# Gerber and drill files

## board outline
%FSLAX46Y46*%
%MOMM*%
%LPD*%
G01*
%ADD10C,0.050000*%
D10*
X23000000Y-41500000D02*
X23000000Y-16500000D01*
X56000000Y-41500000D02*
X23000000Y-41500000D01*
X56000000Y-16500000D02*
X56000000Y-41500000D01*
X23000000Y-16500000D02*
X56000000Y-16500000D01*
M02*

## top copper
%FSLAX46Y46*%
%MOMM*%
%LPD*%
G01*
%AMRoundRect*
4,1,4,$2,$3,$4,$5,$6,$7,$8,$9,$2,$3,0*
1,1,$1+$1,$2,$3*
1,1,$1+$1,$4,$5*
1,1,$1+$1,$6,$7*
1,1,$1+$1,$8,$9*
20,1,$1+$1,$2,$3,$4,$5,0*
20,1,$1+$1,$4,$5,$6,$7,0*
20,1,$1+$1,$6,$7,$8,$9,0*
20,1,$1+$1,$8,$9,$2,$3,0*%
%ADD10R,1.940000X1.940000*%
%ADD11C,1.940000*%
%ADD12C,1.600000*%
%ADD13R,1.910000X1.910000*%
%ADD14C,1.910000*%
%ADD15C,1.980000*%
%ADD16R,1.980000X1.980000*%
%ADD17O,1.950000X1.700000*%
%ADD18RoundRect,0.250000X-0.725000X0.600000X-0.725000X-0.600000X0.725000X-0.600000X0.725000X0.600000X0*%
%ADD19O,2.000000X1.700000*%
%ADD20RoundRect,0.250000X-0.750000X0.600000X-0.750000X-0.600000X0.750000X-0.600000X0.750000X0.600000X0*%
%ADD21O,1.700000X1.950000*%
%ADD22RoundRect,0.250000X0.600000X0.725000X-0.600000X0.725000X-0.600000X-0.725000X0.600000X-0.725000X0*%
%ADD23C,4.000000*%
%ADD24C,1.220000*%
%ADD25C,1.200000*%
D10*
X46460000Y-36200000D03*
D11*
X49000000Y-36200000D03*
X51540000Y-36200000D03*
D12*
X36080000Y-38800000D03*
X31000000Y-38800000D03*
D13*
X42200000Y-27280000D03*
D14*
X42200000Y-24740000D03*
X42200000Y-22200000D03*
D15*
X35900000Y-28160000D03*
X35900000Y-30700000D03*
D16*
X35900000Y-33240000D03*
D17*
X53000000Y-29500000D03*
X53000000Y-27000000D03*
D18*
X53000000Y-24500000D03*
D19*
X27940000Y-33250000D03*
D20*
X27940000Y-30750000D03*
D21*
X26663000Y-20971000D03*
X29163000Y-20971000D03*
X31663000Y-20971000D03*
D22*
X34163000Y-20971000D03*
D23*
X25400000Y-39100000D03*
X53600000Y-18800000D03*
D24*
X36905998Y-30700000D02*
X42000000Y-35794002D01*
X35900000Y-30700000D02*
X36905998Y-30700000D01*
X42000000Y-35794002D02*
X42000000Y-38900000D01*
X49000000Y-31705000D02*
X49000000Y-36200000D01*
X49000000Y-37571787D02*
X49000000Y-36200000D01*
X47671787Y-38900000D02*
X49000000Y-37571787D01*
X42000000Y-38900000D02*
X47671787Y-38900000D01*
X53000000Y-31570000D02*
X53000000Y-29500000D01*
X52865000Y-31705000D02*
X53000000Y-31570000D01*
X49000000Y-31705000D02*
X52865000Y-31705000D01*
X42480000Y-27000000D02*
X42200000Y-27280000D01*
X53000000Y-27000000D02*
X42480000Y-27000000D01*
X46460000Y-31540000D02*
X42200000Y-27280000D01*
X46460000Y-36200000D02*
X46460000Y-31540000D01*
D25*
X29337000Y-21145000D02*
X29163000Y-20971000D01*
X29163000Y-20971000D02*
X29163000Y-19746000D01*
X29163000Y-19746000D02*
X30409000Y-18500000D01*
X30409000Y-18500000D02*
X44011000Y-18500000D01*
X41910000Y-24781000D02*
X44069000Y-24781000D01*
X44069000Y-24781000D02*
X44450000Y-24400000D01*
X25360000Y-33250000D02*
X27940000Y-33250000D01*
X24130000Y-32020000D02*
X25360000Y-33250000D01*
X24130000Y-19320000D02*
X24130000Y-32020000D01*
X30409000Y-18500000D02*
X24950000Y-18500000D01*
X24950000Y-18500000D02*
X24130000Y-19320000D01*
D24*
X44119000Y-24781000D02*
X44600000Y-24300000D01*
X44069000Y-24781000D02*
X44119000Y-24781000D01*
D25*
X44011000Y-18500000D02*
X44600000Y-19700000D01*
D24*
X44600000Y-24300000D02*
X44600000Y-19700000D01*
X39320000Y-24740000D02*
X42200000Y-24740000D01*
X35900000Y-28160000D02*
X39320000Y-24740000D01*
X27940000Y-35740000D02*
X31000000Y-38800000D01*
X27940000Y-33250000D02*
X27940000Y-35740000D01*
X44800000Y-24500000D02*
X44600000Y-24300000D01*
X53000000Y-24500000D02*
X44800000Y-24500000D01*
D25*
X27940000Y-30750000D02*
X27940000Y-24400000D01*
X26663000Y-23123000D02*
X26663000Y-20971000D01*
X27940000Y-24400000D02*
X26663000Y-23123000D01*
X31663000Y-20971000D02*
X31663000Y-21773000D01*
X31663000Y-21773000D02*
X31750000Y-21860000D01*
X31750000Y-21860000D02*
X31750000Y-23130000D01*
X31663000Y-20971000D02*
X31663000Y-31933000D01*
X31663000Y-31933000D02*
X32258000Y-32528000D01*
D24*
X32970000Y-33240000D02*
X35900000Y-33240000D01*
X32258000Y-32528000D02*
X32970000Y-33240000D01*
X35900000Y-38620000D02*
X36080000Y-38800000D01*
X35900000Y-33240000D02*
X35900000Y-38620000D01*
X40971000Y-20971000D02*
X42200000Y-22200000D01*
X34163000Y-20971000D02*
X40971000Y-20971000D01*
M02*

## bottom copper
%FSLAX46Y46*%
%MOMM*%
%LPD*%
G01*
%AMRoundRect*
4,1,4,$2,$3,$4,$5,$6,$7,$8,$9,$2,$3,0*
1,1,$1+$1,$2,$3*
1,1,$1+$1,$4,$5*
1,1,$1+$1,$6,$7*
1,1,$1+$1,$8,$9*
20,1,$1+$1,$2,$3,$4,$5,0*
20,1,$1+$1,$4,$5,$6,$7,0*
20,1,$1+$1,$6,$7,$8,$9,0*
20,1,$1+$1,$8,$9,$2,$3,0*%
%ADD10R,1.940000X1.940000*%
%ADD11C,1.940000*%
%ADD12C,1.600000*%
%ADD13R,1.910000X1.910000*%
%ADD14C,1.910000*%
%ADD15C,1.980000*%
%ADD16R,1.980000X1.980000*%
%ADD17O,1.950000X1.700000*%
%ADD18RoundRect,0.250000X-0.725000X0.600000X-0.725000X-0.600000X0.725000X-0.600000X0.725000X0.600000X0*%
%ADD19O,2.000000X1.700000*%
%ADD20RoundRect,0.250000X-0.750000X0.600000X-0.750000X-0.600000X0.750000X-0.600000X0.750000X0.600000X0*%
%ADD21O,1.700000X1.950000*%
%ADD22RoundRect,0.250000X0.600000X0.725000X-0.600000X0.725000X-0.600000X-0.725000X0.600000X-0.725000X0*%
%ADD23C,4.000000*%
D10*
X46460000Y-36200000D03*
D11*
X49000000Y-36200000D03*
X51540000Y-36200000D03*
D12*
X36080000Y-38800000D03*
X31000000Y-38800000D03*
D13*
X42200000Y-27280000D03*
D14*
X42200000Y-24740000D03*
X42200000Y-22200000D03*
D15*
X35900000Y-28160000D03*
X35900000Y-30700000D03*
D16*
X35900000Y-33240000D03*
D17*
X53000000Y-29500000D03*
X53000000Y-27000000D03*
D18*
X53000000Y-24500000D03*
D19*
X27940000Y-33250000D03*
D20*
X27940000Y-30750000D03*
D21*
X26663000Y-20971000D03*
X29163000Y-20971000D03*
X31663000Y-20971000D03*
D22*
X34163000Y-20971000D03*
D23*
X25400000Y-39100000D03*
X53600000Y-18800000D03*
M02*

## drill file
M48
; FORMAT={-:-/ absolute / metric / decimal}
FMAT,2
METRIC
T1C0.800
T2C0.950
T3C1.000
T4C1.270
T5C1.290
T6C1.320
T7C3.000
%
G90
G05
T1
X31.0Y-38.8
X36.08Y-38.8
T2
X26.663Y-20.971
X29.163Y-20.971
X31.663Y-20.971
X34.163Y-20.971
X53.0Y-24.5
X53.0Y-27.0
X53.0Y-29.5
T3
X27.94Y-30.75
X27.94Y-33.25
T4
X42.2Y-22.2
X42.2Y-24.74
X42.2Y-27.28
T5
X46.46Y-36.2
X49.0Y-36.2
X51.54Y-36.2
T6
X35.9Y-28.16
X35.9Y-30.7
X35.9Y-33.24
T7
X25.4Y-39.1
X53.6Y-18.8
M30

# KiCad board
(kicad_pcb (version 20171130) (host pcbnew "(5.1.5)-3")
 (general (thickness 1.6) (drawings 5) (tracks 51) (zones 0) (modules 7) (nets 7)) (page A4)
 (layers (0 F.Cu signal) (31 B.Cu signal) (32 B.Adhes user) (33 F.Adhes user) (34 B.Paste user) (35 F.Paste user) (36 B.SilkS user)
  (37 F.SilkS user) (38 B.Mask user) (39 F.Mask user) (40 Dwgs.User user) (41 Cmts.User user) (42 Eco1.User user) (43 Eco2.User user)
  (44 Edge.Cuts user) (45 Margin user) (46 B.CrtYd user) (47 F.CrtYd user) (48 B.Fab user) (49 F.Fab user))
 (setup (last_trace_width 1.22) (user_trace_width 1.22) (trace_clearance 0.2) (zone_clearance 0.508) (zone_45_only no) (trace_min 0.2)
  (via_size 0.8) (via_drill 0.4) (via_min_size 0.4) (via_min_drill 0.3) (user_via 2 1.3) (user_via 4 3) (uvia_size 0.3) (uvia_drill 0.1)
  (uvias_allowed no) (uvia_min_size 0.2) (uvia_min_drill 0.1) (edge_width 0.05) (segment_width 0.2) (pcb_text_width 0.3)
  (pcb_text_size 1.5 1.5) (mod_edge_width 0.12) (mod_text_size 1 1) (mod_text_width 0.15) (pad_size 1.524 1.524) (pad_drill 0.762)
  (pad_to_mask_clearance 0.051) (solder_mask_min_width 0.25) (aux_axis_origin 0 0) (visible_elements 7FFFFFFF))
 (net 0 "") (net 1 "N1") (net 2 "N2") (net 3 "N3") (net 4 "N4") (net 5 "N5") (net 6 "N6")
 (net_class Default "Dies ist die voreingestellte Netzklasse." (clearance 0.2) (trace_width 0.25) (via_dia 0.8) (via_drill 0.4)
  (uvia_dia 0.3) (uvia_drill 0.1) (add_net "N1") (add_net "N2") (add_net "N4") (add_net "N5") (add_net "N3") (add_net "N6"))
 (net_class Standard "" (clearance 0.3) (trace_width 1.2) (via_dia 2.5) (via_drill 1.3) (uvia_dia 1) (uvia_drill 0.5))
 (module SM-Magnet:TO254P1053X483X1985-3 (layer F.Cu) (at 49 36.2)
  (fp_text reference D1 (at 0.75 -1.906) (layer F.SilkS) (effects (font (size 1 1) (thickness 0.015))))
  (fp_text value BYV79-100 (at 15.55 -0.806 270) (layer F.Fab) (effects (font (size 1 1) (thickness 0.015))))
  (pad 1 thru_hole rect (at -2.54 0) (size 1.94 1.94) (drill 1.29) (layers *.Cu *.Mask) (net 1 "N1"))
  (pad 2 thru_hole circle (at 0 0) (size 1.94 1.94) (drill 1.29) (layers *.Cu *.Mask) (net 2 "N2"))
  (pad 3 thru_hole circle (at 2.54 0) (size 1.94 1.94) (drill 1.29) (layers *.Cu *.Mask)))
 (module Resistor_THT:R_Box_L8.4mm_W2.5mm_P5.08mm (layer F.Cu) (at 31 38.8)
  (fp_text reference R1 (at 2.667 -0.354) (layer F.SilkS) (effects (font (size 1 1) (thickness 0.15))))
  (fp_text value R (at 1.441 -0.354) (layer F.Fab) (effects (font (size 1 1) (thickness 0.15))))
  (pad 2 thru_hole circle (at 5.08 0) (size 1.6 1.6) (drill 0.8) (layers *.Cu *.Mask) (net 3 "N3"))
  (pad 1 thru_hole circle (at 0 0) (size 1.6 1.6) (drill 0.8) (layers *.Cu *.Mask) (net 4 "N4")))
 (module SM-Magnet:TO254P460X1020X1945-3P (layer F.Cu) (at 42.2 24.74 180)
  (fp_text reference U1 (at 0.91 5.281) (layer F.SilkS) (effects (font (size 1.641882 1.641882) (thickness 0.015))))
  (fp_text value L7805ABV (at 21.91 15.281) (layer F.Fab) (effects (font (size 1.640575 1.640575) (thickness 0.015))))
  (pad 1 thru_hole rect (at 0 -2.54 180) (size 1.91 1.91) (drill 1.27) (layers *.Cu *.Mask) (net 1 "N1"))
  (pad 2 thru_hole circle (at 0 0 180) (size 1.91 1.91) (drill 1.27) (layers *.Cu *.Mask) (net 4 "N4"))
  (pad 3 thru_hole circle (at 0 2.54 180) (size 1.91 1.91) (drill 1.27) (layers *.Cu *.Mask) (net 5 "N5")))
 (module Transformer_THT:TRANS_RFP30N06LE (layer F.Cu) (at 35.9 30.7 90)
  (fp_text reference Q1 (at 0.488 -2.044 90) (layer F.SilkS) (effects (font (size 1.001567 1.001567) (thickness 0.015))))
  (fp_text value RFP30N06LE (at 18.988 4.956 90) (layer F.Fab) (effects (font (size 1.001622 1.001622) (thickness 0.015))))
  (pad 3 thru_hole circle (at 2.54 0 90) (size 1.98 1.98) (drill 1.32) (layers *.Cu *.Mask) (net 4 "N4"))
  (pad 2 thru_hole circle (at 0 0 90) (size 1.98 1.98) (drill 1.32) (layers *.Cu *.Mask) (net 2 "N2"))
  (pad 1 thru_hole rect (at -2.54 0 90) (size 1.98 1.98) (drill 1.32) (layers *.Cu *.Mask) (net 3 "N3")))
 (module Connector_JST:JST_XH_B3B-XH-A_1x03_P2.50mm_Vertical (layer F.Cu) (at 53 24.5 270)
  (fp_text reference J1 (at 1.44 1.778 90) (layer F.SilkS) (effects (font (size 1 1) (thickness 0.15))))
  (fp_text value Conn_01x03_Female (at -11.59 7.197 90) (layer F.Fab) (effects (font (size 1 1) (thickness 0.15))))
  (pad 3 thru_hole oval (at 5 0 270) (size 1.7 1.95) (drill 0.95) (layers *.Cu *.Mask) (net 2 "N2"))
  (pad 2 thru_hole oval (at 2.5 0 270) (size 1.7 1.95) (drill 0.95) (layers *.Cu *.Mask) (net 1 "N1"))
  (pad 1 thru_hole roundrect (at 0 0 270) (size 1.7 1.95) (drill 0.95) (layers *.Cu *.Mask) (roundrect_rratio 0.147059) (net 4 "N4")))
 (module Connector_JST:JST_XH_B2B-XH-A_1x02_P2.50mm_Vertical (layer F.Cu) (at 27.94 30.75 270)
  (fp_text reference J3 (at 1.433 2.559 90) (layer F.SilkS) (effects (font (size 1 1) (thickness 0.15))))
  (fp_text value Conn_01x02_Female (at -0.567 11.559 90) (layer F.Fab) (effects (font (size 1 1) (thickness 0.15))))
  (pad 2 thru_hole oval (at 2.5 0 270) (size 1.7 2) (drill 1) (layers *.Cu *.Mask) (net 4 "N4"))
  (pad 1 thru_hole roundrect (at 0 0 270) (size 1.7 2) (drill 1) (layers *.Cu *.Mask) (roundrect_rratio 0.147059) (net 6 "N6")))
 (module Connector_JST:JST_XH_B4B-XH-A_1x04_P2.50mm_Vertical (layer F.Cu) (at 34.163 20.971 180)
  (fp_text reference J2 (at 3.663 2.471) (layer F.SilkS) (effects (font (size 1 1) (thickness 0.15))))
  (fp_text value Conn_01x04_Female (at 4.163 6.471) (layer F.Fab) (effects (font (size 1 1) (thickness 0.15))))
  (pad 4 thru_hole oval (at 7.5 0 180) (size 1.7 1.95) (drill 0.95) (layers *.Cu *.Mask) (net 6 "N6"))
  (pad 3 thru_hole oval (at 5 0 180) (size 1.7 1.95) (drill 0.95) (layers *.Cu *.Mask) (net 4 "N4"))
  (pad 2 thru_hole oval (at 2.5 0 180) (size 1.7 1.95) (drill 0.95) (layers *.Cu *.Mask) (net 3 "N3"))
  (pad 1 thru_hole roundrect (at 0 0 180) (size 1.7 1.95) (drill 0.95) (layers *.Cu *.Mask) (roundrect_rratio 0.147059) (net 5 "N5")))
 (gr_line (start 23 41.5) (end 23 16.5) (layer Edge.Cuts) (width 0.05))
 (gr_line (start 56 41.5) (end 23 41.5) (layer Edge.Cuts) (width 0.05))
 (gr_line (start 56 16.5) (end 56 41.5) (layer Edge.Cuts) (width 0.05))
 (gr_line (start 23 16.5) (end 56 16.5) (layer Edge.Cuts) (width 0.05))
 (via (at 25.4 39.1) (size 4) (drill 3) (layers F.Cu B.Cu) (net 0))
 (via (at 53.6 18.8) (size 4) (drill 3) (layers F.Cu B.Cu) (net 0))
 (segment (start 36.905998 30.7) (end 42 35.794002) (width 1.22) (layer F.Cu) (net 2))
 (segment (start 35.9 30.7) (end 36.905998 30.7) (width 1.22) (layer F.Cu) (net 2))
 (segment (start 42 35.794002) (end 42 38.9) (width 1.22) (layer F.Cu) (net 2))
 (segment (start 49 31.705) (end 49 36.2) (width 1.22) (layer F.Cu) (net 2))
 (segment (start 49 37.571787) (end 49 36.2) (width 1.22) (layer F.Cu) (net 2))
 (segment (start 47.671787 38.9) (end 49 37.571787) (width 1.22) (layer F.Cu) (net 2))
 (segment (start 42 38.9) (end 47.671787 38.9) (width 1.22) (layer F.Cu) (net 2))
 (segment (start 53 31.57) (end 53 29.5) (width 1.22) (layer F.Cu) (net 2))
 (segment (start 52.865 31.705) (end 53 31.57) (width 1.22) (layer F.Cu) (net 2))
 (segment (start 49 31.705) (end 52.865 31.705) (width 1.22) (layer F.Cu) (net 2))
 (segment (start 42.48 27) (end 42.2 27.28) (width 1.22) (layer F.Cu) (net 1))
 (segment (start 53 27) (end 42.48 27) (width 1.22) (layer F.Cu) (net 1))
 (segment (start 46.46 31.54) (end 42.2 27.28) (width 1.22) (layer F.Cu) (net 1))
 (segment (start 46.46 36.2) (end 46.46 31.54) (width 1.22) (layer F.Cu) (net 1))
 (segment (start 29.337 21.145) (end 29.163 20.971) (width 1.2) (layer F.Cu) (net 4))
 (segment (start 29.163 20.971) (end 29.163 19.746) (width 1.2) (layer F.Cu) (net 4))
 (segment (start 29.163 19.746) (end 30.409 18.5) (width 1.2) (layer F.Cu) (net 4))
 (segment (start 30.409 18.5) (end 44.011 18.5) (width 1.2) (layer F.Cu) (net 4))
 (segment (start 41.91 24.781) (end 44.069 24.781) (width 1.2) (layer F.Cu) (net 4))
 (segment (start 44.069 24.781) (end 44.45 24.4) (width 1.2) (layer F.Cu) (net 4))
 (segment (start 25.36 33.25) (end 27.94 33.25) (width 1.2) (layer F.Cu) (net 4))
 (segment (start 24.13 32.02) (end 25.36 33.25) (width 1.2) (layer F.Cu) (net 4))
 (segment (start 24.13 19.32) (end 24.13 32.02) (width 1.2) (layer F.Cu) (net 4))
 (segment (start 30.409 18.5) (end 24.95 18.5) (width 1.2) (layer F.Cu) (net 4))
 (segment (start 24.95 18.5) (end 24.13 19.32) (width 1.2) (layer F.Cu) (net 4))
 (segment (start 44.119 24.781) (end 44.6 24.3) (width 1.22) (layer F.Cu) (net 4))
 (segment (start 44.069 24.781) (end 44.119 24.781) (width 1.22) (layer F.Cu) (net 4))
 (segment (start 44.011 18.5) (end 44.6 19.7) (width 1.2) (layer F.Cu) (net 4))
 (segment (start 44.6 24.3) (end 44.6 19.7) (width 1.22) (layer F.Cu) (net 4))
 (segment (start 39.32 24.74) (end 42.2 24.74) (width 1.22) (layer F.Cu) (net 4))
 (segment (start 35.9 28.16) (end 39.32 24.74) (width 1.22) (layer F.Cu) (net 4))
 (segment (start 27.94 35.74) (end 31 38.8) (width 1.22) (layer F.Cu) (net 4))
 (segment (start 27.94 33.25) (end 27.94 35.74) (width 1.22) (layer F.Cu) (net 4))
 (segment (start 44.8 24.5) (end 44.6 24.3) (width 1.22) (layer F.Cu) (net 4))
 (segment (start 53 24.5) (end 44.8 24.5) (width 1.22) (layer F.Cu) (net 4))
 (segment (start 27.94 30.75) (end 27.94 24.4) (width 1.2) (layer F.Cu) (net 6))
 (segment (start 26.663 23.123) (end 26.663 20.971) (width 1.2) (layer F.Cu) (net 6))
 (segment (start 27.94 24.4) (end 26.663 23.123) (width 1.2) (layer F.Cu) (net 6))
 (segment (start 31.663 20.971) (end 31.663 21.773) (width 1.2) (layer F.Cu) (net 3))
 (segment (start 31.663 21.773) (end 31.75 21.86) (width 1.2) (layer F.Cu) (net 3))
 (segment (start 31.75 21.86) (end 31.75 23.13) (width 1.2) (layer F.Cu) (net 3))
 (segment (start 31.663 20.971) (end 31.663 31.933) (width 1.2) (layer F.Cu) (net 3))
 (segment (start 31.663 31.933) (end 32.258 32.528) (width 1.2) (layer F.Cu) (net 3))
 (segment (start 32.97 33.24) (end 35.9 33.24) (width 1.22) (layer F.Cu) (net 3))
 (segment (start 32.258 32.528) (end 32.97 33.24) (width 1.22) (layer F.Cu) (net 3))
 (segment (start 35.9 38.62) (end 36.08 38.8) (width 1.22) (layer F.Cu) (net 3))
 (segment (start 35.9 33.24) (end 35.9 38.62) (width 1.22) (layer F.Cu) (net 3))
 (segment (start 40.971 20.971) (end 42.2 22.2) (width 1.22) (layer F.Cu) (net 5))
 (segment (start 34.163 20.971) (end 40.971 20.971) (width 1.22) (layer F.Cu) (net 5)))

